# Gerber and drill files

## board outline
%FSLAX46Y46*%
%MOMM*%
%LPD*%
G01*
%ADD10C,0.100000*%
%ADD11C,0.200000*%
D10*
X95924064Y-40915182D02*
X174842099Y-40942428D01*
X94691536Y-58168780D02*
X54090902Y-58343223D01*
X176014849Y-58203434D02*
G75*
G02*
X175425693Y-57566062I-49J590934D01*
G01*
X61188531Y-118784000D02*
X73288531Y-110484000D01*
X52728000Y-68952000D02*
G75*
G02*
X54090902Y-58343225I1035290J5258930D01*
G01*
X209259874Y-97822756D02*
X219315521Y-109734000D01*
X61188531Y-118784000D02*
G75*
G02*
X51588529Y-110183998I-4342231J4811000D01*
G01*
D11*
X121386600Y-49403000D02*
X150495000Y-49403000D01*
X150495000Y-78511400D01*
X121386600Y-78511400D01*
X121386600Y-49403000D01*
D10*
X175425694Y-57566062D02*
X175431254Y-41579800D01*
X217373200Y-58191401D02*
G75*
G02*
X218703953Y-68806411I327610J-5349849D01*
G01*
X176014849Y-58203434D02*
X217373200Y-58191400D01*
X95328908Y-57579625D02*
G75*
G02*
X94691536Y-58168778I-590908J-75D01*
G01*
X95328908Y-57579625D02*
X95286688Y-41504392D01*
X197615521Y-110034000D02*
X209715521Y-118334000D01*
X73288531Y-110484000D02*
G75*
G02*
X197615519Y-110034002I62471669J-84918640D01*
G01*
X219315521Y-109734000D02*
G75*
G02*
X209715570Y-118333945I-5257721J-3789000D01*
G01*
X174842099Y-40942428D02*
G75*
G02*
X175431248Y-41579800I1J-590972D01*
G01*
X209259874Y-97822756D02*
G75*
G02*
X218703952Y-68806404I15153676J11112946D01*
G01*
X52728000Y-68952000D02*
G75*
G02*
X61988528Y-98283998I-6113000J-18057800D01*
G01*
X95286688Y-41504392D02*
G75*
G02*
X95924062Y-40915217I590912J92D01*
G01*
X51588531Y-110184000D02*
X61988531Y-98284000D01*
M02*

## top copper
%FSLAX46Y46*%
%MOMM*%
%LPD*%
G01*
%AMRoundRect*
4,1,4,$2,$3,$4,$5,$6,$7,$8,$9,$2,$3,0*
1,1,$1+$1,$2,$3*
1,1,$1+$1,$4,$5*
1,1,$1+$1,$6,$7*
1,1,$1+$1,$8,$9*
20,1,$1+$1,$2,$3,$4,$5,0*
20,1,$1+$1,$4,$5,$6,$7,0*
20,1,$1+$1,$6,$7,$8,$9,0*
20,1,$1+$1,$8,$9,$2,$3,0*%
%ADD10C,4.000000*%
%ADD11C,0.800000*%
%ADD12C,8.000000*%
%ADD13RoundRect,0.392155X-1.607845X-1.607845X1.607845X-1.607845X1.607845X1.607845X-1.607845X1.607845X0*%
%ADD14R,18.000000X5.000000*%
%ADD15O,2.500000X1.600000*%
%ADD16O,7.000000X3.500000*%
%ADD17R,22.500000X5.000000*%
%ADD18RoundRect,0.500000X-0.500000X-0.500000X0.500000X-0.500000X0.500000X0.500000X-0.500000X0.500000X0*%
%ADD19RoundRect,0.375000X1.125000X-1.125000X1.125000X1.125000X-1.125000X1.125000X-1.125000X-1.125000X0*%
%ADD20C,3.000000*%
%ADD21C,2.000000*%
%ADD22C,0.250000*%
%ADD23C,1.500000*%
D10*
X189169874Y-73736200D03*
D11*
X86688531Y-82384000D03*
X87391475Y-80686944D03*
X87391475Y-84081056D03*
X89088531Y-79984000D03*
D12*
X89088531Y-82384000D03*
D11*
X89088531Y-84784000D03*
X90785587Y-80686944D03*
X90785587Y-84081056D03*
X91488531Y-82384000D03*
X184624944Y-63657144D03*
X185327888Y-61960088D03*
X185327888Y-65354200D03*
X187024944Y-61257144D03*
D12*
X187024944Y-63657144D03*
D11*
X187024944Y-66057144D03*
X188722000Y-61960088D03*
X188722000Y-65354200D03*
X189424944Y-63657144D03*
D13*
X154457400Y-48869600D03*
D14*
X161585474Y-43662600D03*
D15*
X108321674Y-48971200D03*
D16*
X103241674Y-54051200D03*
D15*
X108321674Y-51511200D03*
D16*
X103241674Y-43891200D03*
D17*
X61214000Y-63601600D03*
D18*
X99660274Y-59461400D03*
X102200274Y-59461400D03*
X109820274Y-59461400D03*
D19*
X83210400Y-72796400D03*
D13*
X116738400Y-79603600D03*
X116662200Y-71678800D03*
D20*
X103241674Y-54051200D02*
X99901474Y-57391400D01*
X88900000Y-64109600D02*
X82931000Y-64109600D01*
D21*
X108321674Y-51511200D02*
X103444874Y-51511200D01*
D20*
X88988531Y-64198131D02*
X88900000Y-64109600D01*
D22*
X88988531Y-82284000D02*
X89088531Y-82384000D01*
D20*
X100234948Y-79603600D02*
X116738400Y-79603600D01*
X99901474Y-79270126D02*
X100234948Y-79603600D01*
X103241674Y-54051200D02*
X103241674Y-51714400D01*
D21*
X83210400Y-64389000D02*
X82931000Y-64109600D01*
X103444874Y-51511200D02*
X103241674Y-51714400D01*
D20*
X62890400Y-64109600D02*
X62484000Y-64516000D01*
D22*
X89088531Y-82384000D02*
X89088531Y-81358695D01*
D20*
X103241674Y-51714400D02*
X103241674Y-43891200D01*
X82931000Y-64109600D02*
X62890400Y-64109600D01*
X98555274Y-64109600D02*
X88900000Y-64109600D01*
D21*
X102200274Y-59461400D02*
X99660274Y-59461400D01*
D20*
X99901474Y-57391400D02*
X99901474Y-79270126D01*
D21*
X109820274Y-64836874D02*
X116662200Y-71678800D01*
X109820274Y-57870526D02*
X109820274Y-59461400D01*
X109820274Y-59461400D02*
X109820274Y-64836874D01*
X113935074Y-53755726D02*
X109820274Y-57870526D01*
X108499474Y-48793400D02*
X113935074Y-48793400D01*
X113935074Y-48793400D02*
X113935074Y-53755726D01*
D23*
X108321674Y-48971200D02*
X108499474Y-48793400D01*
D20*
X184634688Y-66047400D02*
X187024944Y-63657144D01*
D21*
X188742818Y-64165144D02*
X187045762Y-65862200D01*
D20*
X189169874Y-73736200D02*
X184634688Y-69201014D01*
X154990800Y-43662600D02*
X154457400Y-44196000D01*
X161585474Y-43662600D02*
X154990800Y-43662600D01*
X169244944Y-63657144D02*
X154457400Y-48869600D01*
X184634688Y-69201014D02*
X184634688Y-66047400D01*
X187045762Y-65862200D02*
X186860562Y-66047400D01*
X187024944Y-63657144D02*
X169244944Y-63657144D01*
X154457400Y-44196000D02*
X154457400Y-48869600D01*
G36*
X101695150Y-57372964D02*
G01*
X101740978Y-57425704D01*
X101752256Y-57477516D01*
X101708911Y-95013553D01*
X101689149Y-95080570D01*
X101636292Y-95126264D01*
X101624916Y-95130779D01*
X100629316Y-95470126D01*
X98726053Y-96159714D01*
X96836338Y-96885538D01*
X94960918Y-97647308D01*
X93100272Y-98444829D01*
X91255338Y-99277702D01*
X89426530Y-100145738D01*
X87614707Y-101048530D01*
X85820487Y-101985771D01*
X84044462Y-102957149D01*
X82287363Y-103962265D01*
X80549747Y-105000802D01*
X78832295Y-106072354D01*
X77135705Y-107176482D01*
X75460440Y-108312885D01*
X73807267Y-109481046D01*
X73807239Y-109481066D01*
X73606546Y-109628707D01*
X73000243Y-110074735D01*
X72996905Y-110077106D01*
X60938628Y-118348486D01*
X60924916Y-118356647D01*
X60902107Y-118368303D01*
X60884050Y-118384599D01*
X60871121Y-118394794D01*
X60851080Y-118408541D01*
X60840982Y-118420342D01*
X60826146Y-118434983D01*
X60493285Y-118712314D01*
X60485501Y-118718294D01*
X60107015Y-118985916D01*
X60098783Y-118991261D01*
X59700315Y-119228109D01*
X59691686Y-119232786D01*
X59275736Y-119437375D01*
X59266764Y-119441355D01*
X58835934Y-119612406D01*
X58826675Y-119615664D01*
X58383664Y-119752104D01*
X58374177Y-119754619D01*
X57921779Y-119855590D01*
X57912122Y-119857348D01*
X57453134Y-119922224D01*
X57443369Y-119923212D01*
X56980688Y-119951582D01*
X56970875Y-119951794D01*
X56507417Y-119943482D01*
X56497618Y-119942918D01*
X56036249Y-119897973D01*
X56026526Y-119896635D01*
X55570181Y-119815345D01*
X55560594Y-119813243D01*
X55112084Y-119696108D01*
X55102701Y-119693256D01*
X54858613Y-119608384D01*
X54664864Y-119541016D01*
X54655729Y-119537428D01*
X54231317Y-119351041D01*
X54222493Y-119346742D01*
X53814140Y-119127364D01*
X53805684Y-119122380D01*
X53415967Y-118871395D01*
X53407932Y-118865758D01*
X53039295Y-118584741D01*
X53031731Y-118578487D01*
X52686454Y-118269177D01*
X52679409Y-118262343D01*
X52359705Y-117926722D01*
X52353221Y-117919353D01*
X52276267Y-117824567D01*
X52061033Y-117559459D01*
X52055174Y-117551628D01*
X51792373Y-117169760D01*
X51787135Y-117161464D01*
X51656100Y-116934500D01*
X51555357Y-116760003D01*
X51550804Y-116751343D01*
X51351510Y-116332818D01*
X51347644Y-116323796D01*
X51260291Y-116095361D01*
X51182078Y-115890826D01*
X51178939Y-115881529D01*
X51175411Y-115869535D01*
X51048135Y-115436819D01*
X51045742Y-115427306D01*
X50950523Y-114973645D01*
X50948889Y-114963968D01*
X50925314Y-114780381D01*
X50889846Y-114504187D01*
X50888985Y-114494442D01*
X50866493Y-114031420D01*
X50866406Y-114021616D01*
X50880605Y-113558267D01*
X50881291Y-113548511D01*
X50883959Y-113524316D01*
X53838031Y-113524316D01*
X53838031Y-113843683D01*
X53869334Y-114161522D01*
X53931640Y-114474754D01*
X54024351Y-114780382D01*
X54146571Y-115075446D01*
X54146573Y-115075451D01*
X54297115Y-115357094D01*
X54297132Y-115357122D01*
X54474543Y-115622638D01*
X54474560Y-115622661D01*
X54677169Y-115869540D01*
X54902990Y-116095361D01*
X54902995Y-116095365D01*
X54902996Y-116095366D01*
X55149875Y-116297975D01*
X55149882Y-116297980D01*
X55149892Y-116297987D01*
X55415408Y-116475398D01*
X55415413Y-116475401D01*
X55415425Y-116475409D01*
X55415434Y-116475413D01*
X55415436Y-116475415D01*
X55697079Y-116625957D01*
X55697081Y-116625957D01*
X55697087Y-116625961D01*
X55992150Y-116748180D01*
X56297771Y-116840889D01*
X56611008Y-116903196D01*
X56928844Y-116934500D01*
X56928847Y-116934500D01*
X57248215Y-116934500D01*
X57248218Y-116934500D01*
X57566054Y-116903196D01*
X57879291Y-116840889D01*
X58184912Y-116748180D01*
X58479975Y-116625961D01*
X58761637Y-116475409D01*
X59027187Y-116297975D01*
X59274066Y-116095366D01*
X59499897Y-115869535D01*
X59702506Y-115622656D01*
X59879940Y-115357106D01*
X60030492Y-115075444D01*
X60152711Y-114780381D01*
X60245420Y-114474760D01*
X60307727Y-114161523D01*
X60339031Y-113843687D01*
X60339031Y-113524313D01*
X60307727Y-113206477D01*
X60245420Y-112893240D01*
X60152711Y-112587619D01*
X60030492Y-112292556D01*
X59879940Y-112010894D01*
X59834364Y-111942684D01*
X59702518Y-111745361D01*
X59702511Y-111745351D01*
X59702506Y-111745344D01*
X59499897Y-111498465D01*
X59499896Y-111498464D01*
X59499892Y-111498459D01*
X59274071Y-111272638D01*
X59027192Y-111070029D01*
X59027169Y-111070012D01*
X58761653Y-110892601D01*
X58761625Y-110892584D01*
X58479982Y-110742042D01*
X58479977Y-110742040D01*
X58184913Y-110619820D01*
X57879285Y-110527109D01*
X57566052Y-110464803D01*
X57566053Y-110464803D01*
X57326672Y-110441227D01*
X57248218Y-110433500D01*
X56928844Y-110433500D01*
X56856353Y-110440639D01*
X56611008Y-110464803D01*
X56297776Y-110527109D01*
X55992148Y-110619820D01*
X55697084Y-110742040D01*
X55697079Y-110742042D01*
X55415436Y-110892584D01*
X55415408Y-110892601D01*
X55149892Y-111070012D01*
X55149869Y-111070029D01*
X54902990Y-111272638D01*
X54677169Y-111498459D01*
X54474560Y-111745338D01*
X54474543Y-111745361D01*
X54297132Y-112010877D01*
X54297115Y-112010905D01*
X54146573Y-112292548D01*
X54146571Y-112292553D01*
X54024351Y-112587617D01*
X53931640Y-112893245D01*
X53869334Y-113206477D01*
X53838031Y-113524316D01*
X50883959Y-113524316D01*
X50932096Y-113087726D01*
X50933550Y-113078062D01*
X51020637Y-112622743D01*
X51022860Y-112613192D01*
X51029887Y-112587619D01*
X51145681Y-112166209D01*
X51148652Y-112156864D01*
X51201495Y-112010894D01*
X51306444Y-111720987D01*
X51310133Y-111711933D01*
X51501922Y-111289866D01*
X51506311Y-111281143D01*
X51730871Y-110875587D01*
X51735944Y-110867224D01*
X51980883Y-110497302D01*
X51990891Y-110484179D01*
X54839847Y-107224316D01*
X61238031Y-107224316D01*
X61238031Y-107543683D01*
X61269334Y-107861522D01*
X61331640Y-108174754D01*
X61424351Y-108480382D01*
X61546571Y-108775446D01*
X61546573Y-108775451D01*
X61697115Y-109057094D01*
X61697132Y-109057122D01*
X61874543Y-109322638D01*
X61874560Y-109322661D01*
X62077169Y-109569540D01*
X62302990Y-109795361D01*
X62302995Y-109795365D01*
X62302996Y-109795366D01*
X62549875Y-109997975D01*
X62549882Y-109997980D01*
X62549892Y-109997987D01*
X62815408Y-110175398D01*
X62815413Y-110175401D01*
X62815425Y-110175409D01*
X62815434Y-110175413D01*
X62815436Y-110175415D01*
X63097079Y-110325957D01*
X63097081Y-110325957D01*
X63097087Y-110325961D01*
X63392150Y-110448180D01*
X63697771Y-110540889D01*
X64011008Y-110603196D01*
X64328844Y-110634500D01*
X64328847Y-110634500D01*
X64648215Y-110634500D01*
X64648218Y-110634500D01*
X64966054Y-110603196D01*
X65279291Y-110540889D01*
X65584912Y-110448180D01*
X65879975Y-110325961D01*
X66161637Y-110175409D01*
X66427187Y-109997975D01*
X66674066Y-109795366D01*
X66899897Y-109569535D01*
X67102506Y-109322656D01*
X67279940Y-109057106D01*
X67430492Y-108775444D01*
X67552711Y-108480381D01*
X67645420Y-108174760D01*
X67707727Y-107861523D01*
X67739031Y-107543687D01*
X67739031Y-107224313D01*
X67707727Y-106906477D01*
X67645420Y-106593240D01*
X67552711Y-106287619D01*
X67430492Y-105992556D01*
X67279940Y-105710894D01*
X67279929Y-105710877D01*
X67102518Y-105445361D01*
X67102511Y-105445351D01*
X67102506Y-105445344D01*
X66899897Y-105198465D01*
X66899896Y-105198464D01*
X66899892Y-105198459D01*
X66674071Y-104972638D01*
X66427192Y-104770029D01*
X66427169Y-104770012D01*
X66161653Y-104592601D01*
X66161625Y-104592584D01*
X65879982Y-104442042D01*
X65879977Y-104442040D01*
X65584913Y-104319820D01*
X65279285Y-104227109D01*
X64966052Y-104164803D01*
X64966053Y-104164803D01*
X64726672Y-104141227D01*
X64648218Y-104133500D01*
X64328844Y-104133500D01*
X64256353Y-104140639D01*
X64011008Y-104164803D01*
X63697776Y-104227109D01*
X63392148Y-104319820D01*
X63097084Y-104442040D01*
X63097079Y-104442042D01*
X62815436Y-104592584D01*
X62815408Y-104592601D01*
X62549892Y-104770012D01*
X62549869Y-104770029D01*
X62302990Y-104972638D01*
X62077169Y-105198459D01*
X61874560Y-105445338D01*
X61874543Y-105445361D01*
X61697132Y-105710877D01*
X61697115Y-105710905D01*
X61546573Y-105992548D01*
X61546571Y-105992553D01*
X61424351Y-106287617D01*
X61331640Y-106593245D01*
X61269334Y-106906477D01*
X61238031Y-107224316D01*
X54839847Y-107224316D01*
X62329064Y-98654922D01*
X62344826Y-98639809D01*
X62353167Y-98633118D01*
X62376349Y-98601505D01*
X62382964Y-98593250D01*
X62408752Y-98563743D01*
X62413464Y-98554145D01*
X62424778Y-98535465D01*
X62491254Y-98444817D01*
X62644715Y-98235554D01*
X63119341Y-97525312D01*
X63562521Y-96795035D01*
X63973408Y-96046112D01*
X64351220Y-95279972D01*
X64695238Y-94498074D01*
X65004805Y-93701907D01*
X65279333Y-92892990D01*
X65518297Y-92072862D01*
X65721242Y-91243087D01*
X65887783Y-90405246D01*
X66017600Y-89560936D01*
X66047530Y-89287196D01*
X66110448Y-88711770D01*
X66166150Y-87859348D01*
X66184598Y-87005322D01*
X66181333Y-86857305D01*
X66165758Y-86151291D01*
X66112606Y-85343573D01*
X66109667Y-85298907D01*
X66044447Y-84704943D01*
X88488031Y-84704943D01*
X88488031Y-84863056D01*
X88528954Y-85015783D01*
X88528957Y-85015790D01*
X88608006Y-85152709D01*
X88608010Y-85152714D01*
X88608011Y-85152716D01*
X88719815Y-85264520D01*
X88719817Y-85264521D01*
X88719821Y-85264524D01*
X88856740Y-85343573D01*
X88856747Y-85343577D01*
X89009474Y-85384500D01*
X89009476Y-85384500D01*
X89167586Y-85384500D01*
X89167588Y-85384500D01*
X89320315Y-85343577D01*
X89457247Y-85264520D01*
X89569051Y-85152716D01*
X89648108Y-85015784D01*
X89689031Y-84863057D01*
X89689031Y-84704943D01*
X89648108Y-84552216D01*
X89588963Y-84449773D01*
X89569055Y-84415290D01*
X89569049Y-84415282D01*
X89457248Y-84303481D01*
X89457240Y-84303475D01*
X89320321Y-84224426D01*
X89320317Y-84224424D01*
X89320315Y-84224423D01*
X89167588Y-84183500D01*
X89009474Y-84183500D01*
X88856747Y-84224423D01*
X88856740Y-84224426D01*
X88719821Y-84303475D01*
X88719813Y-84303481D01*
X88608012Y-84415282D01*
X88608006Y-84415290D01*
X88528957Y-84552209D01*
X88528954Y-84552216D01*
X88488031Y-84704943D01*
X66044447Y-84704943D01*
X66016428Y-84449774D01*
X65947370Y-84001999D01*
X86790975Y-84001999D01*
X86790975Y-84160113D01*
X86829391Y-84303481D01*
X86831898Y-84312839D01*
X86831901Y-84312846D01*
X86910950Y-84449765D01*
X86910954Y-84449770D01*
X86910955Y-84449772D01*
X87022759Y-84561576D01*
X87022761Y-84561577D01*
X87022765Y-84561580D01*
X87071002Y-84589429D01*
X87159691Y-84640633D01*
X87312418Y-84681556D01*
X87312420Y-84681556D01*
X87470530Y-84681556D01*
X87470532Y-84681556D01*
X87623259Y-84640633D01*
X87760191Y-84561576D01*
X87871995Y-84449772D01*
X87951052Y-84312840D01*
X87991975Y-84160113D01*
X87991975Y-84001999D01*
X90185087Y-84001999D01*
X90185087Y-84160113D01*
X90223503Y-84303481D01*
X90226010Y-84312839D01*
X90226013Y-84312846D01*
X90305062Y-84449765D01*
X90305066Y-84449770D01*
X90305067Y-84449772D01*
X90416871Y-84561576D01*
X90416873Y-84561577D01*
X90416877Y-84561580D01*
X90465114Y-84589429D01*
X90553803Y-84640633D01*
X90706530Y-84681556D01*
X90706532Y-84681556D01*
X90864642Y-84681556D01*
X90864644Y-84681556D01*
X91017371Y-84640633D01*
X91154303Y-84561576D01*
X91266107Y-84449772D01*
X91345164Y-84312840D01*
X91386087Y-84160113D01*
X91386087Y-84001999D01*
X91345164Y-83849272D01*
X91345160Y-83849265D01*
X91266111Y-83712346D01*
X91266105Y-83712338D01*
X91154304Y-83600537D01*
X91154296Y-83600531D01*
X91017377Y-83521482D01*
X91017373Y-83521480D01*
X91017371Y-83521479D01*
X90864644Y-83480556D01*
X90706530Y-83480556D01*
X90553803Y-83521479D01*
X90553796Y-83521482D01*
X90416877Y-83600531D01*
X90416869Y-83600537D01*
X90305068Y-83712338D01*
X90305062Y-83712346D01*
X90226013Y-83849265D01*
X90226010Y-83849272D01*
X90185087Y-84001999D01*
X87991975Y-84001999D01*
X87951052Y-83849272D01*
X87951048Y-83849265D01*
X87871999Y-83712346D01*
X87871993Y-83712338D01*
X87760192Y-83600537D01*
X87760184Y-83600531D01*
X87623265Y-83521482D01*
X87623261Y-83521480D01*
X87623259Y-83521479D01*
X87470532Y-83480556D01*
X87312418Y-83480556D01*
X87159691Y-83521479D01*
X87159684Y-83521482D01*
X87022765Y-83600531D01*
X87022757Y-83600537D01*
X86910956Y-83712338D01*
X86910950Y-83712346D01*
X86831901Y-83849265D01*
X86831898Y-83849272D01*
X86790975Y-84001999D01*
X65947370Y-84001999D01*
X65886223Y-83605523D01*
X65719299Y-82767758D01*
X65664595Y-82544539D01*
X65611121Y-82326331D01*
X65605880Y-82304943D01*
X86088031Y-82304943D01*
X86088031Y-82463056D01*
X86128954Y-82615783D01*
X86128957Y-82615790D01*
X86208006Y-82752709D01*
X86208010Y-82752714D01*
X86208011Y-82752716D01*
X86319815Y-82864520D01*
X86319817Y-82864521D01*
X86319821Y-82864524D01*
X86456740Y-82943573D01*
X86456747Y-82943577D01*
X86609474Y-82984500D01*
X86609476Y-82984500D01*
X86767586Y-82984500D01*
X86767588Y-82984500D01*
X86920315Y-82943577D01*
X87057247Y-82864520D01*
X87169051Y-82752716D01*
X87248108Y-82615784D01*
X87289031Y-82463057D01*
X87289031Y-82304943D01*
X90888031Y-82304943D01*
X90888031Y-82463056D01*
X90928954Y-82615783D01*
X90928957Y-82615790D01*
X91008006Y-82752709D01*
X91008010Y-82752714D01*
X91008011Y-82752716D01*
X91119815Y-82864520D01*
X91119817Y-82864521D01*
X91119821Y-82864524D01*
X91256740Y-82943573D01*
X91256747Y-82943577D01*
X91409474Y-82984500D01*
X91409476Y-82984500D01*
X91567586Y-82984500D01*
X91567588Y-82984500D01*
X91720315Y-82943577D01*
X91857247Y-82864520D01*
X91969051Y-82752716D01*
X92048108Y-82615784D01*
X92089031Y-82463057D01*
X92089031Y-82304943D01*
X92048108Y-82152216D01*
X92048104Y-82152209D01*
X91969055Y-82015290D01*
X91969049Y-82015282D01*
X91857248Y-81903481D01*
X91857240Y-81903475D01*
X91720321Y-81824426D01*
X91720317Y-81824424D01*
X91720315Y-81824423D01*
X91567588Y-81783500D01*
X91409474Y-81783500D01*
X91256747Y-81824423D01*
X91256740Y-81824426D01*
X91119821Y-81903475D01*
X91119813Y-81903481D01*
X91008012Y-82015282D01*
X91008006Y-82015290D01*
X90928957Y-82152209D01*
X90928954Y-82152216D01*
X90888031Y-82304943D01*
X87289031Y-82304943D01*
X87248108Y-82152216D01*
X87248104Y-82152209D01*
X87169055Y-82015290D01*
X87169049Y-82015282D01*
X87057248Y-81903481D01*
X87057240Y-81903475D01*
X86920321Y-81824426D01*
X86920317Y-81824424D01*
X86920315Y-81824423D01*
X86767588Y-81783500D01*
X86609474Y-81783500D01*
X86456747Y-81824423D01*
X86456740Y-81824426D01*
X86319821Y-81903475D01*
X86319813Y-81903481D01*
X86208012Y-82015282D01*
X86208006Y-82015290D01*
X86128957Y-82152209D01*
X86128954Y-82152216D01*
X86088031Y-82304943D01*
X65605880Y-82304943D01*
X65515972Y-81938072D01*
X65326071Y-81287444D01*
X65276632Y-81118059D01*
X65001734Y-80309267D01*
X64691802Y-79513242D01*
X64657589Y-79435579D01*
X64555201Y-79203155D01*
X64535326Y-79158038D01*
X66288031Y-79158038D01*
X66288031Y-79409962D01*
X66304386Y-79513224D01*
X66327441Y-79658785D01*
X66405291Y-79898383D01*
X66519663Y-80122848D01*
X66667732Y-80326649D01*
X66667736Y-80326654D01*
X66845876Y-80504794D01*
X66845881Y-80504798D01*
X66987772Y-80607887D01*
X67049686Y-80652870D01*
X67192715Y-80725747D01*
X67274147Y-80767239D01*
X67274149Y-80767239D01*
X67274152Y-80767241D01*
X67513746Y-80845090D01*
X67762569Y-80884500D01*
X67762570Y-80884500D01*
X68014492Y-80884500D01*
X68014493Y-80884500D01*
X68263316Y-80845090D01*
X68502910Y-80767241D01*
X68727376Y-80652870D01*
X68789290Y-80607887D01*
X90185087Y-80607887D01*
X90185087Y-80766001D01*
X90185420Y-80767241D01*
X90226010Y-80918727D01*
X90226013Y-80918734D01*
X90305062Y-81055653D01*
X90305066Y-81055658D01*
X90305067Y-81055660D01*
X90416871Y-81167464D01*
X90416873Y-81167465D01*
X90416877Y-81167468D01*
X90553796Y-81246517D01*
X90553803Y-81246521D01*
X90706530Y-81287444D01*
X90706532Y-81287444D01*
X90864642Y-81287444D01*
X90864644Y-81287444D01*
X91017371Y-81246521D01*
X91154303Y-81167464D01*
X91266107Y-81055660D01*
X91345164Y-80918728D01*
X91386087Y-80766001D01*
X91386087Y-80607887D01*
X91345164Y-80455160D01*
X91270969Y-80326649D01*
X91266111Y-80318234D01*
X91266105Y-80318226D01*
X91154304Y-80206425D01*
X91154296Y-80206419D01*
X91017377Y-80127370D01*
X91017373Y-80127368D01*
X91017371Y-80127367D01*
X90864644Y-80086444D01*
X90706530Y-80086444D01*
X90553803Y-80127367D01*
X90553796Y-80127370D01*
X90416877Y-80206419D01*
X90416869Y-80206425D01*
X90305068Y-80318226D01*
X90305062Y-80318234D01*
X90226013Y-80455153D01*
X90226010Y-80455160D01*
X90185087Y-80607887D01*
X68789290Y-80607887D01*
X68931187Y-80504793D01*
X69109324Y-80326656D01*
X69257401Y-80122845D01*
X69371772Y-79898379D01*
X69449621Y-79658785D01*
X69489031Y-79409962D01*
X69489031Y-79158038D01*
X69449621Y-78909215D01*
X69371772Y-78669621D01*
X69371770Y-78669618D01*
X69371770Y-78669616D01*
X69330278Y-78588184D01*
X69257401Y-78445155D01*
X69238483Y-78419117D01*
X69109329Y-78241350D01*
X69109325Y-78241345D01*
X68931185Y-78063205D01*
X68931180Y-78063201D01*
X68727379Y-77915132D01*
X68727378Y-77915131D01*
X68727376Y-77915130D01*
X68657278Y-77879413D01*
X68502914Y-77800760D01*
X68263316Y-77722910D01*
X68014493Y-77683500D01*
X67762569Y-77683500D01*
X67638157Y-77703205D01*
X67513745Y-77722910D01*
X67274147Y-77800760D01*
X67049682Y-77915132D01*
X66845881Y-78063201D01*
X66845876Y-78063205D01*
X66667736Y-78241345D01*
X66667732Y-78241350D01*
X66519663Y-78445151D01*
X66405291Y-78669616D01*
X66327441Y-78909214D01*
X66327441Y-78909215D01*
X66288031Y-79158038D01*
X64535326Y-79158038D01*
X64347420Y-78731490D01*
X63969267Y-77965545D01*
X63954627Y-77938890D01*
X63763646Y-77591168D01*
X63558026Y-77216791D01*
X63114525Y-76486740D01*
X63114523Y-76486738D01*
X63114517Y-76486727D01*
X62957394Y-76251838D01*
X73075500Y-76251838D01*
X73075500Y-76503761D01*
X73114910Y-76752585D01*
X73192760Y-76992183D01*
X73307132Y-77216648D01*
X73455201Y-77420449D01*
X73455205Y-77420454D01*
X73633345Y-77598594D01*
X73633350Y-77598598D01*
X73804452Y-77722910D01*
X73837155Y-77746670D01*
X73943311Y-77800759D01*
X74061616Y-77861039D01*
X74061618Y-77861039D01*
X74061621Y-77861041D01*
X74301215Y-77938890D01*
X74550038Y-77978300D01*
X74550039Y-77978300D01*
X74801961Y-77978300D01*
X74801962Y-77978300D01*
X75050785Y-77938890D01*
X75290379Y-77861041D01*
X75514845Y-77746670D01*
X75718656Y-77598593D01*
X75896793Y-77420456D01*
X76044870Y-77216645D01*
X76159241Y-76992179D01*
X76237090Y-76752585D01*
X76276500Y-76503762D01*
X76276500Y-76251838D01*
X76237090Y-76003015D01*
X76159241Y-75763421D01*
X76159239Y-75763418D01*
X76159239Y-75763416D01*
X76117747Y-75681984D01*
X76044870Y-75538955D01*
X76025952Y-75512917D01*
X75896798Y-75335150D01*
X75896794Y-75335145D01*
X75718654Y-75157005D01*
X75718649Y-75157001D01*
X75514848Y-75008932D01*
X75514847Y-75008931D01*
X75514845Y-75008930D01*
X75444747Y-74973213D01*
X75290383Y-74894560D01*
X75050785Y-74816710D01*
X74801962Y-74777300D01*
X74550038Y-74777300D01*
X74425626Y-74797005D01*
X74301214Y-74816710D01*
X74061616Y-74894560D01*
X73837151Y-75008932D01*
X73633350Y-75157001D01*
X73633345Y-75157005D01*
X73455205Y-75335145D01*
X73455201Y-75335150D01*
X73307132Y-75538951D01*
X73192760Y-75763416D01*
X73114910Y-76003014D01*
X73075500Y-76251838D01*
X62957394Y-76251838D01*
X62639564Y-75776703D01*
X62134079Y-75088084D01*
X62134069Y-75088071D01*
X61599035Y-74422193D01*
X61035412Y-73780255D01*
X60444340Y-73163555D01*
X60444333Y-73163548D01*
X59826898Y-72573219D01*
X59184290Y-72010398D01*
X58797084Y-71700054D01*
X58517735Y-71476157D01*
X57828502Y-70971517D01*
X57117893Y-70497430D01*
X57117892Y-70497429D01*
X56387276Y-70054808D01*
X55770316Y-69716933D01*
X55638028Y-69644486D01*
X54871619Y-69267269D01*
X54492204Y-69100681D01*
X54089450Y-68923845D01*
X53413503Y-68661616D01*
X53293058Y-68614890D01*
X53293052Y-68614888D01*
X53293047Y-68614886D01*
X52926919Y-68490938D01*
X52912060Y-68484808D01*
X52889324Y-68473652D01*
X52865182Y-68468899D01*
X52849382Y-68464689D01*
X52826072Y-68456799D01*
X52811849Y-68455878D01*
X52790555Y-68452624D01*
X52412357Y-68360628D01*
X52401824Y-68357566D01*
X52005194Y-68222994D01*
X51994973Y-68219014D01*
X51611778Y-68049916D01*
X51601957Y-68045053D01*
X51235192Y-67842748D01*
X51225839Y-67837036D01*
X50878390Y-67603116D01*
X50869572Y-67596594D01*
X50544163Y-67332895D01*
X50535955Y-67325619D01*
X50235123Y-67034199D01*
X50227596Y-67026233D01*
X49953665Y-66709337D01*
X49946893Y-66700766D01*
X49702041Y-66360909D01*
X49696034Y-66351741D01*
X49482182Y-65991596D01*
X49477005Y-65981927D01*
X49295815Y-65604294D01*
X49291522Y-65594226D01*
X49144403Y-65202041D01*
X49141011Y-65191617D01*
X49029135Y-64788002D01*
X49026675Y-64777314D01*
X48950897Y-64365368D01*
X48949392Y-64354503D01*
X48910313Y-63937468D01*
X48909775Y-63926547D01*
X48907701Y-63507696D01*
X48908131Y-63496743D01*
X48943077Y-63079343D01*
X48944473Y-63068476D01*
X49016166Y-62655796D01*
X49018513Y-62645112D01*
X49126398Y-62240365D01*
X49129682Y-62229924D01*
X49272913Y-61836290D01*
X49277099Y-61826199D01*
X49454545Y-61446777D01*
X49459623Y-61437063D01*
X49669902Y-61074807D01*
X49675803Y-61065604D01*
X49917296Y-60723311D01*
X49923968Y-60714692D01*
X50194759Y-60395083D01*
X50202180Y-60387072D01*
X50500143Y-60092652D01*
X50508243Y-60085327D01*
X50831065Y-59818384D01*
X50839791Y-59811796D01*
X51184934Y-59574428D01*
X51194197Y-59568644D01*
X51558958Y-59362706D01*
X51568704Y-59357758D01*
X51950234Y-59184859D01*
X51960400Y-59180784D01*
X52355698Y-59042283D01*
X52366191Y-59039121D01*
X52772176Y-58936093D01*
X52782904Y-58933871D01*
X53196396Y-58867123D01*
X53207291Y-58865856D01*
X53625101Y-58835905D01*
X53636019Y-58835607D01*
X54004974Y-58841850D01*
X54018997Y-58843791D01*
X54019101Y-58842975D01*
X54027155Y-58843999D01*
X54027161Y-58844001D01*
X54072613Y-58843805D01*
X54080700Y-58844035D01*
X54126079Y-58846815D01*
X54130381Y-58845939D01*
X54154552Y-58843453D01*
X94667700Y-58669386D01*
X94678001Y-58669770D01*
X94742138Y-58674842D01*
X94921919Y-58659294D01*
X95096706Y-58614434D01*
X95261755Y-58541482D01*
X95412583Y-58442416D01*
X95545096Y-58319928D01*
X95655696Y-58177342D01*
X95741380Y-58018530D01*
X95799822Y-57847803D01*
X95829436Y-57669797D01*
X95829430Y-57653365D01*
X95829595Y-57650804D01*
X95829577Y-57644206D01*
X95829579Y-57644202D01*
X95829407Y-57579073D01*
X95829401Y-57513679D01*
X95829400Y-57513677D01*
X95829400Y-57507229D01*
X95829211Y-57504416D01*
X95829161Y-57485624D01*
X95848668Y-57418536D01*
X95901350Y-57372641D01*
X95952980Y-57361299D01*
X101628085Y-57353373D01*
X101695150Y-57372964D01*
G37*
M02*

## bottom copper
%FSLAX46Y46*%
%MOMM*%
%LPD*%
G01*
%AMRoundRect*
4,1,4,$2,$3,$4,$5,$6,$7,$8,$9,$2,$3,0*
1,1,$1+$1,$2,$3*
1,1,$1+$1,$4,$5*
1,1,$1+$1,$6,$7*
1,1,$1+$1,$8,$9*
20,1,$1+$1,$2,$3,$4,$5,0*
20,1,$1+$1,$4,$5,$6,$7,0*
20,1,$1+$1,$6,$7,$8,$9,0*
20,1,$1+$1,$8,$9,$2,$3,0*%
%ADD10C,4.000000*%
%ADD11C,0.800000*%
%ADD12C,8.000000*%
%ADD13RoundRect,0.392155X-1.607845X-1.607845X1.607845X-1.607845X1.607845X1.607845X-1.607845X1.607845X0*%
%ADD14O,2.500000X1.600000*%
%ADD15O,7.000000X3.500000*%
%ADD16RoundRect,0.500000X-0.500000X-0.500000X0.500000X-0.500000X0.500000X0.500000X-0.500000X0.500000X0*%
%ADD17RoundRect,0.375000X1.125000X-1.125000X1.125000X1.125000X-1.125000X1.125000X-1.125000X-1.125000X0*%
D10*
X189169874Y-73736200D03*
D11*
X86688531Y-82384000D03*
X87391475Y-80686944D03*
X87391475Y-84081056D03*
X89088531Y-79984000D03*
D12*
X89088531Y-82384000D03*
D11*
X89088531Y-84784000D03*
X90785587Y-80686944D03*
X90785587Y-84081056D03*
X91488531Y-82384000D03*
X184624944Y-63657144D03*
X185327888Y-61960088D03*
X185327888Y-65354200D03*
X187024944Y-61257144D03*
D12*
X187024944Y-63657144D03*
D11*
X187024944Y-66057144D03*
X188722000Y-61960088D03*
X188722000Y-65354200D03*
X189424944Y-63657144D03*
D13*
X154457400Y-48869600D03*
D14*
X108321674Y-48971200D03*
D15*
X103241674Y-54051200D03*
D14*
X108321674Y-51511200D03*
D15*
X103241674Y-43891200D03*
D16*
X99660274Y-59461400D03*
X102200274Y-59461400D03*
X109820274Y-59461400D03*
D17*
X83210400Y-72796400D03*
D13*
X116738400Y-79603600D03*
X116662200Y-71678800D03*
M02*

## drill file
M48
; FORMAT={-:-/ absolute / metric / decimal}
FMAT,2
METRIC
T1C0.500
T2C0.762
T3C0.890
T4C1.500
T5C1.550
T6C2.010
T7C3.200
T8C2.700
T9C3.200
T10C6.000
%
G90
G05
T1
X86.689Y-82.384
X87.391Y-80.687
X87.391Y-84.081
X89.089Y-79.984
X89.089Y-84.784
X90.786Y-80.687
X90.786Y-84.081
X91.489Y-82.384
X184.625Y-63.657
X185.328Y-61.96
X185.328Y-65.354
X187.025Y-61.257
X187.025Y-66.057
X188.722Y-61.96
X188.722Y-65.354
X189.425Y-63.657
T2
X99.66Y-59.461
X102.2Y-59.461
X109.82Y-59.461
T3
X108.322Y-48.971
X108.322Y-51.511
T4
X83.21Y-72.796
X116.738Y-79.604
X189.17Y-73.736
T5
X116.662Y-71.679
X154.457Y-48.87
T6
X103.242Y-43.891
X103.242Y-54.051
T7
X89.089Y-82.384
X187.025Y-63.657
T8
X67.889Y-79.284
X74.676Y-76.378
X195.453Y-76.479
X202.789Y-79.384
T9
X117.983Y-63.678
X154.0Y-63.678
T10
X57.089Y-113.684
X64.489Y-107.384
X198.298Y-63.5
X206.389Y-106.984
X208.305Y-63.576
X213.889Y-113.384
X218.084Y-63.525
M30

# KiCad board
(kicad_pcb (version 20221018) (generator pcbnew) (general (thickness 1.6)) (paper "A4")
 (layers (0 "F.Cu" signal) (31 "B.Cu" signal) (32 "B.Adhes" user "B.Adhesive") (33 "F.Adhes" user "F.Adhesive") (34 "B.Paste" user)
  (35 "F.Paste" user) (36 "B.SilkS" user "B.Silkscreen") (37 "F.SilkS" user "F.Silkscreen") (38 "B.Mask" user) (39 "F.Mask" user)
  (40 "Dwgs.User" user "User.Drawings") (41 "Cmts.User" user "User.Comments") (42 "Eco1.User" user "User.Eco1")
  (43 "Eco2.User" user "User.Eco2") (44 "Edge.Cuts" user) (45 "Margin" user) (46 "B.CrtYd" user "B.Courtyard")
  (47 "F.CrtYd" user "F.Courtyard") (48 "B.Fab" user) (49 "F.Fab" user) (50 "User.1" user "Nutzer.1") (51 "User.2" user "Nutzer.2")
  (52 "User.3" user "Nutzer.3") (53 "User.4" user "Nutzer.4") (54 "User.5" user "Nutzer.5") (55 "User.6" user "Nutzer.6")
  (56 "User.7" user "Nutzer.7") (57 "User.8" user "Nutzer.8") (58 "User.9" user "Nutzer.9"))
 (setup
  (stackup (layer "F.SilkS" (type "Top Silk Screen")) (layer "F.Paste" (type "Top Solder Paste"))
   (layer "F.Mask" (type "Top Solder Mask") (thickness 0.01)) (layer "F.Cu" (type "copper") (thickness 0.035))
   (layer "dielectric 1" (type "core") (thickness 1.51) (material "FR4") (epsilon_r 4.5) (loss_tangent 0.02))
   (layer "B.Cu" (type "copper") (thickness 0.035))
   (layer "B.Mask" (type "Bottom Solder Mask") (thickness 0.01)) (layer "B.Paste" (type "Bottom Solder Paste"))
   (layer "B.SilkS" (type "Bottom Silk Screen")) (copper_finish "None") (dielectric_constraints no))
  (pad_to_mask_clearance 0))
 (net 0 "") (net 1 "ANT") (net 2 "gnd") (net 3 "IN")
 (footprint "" (layer "F.Cu") (at 189.169874 73.7362)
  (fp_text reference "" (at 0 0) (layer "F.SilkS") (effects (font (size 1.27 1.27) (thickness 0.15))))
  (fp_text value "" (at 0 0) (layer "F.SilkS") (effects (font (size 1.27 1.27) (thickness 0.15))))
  (pad "1" thru_hole circle (at 0 0 90) (size 4 4) (drill 1.5) (layers "*.Cu" "*.Mask") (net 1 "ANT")))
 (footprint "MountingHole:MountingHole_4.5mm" (layer "F.Cu") (at 218.0844 63.5254)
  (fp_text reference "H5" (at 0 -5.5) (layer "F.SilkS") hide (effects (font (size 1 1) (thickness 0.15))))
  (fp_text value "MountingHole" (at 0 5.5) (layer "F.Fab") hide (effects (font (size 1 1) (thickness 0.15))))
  (pad "" np_thru_hole circle (at 0 0) (size 6 6) (drill 6) (layers "F&B.Cu" "*.Mask")))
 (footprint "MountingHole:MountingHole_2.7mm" (layer "F.Cu") (at 195.453 76.4794)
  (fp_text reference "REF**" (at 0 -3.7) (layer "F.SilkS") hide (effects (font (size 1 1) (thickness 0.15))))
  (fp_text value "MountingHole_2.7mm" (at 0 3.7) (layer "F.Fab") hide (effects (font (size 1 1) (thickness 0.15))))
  (pad "" np_thru_hole circle (at 0 0) (size 2.7 2.7) (drill 2.7) (layers "F&B.Cu" "*.Mask")))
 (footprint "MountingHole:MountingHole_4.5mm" (layer "F.Cu") (at 198.2978 63.5)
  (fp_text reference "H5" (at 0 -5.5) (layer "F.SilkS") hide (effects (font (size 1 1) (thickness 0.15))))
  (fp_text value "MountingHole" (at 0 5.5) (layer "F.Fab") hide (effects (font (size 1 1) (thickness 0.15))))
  (pad "" np_thru_hole circle (at 0 0) (size 6 6) (drill 6) (layers "F&B.Cu" "*.Mask")))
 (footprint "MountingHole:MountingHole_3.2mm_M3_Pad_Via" (layer "F.Cu") (at 89.088531 82.384)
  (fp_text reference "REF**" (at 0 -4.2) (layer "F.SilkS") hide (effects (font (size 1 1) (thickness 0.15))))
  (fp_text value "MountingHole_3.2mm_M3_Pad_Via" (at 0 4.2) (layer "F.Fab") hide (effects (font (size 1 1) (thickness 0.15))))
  (pad "1" thru_hole circle (at -2.4 0) (size 0.8 0.8) (drill 0.5) (layers "*.Cu" "*.Mask"))
  (pad "1" thru_hole circle (at -1.697056 -1.697056) (size 0.8 0.8) (drill 0.5) (layers "*.Cu" "*.Mask") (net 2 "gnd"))
  (pad "1" thru_hole circle (at -1.697056 1.697056) (size 0.8 0.8) (drill 0.5) (layers "*.Cu" "*.Mask"))
  (pad "1" thru_hole circle (at 0 -2.4) (size 0.8 0.8) (drill 0.5) (layers "*.Cu" "*.Mask") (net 2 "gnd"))
  (pad "1" thru_hole circle (at 0 0) (size 8 8) (drill 3.2) (layers "*.Cu" "*.Mask") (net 2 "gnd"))
  (pad "1" thru_hole circle (at 0 2.4) (size 0.8 0.8) (drill 0.5) (layers "*.Cu" "*.Mask"))
  (pad "1" thru_hole circle (at 1.697056 -1.697056) (size 0.8 0.8) (drill 0.5) (layers "*.Cu" "*.Mask"))
  (pad "1" thru_hole circle (at 1.697056 1.697056) (size 0.8 0.8) (drill 0.5) (layers "*.Cu" "*.Mask"))
  (pad "1" thru_hole circle (at 2.4 0) (size 0.8 0.8) (drill 0.5) (layers "*.Cu" "*.Mask")))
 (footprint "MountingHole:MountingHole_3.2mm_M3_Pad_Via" (layer "F.Cu") (at 187.024944 63.657144)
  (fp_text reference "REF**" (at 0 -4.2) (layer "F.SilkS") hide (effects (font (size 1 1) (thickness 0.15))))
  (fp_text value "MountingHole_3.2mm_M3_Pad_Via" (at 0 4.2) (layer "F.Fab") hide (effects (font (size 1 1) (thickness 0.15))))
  (pad "1" thru_hole circle (at -2.4 0) (size 0.8 0.8) (drill 0.5) (layers "*.Cu" "*.Mask") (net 1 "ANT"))
  (pad "1" thru_hole circle (at -1.697056 -1.697056) (size 0.8 0.8) (drill 0.5) (layers "*.Cu" "*.Mask") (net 1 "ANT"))
  (pad "1" thru_hole circle (at -1.697056 1.697056) (size 0.8 0.8) (drill 0.5) (layers "*.Cu" "*.Mask") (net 1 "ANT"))
  (pad "1" thru_hole circle (at 0 -2.4) (size 0.8 0.8) (drill 0.5) (layers "*.Cu" "*.Mask") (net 1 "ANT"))
  (pad "1" thru_hole circle (at 0 0) (size 8 8) (drill 3.2) (layers "*.Cu" "*.Mask") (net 1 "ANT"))
  (pad "1" thru_hole circle (at 0 2.4) (size 0.8 0.8) (drill 0.5) (layers "*.Cu" "*.Mask") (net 1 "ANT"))
  (pad "1" thru_hole circle (at 1.697056 -1.697056) (size 0.8 0.8) (drill 0.5) (layers "*.Cu" "*.Mask") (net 1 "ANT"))
  (pad "1" thru_hole circle (at 1.697056 1.697056) (size 0.8 0.8) (drill 0.5) (layers "*.Cu" "*.Mask") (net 1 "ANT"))
  (pad "1" thru_hole circle (at 2.4 0) (size 0.8 0.8) (drill 0.5) (layers "*.Cu" "*.Mask") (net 1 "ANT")))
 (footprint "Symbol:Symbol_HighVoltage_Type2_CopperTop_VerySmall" (layer "F.Cu") (at 193.0146 68.072)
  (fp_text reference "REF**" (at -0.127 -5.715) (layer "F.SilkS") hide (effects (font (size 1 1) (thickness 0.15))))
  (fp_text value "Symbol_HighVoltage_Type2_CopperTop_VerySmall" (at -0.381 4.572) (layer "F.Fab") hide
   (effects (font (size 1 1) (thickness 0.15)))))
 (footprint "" (layer "F.Cu") (at 154.4574 48.8696)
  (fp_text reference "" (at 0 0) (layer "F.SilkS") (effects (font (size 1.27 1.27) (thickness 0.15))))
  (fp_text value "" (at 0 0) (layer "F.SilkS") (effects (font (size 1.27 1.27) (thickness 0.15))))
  (pad "5" thru_hole roundrect (at 0 0) (size 4 4) (drill 1.55) (layers "*.Cu" "*.Mask") (roundrect_rratio 0.09803875) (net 1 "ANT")))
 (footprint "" (layer "F.Cu") (at 154.0002 63.6778)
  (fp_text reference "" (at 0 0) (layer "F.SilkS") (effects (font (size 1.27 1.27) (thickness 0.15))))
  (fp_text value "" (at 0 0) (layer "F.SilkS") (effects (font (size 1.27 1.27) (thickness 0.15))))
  (pad "" np_thru_hole circle (at 0 0) (size 3.2 3.2) (drill 3.2) (layers "*.Cu" "*.Mask")))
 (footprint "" (layer "F.Cu") (at 161.585474 43.6626)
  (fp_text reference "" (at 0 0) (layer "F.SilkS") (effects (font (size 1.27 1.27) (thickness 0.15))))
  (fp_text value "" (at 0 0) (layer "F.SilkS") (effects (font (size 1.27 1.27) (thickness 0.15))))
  (pad "1" smd rect (at 0 0) (size 18 5) (layers "F.Cu" "F.Mask") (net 1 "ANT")))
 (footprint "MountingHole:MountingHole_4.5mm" (layer "F.Cu") (at 208.3054 63.5762)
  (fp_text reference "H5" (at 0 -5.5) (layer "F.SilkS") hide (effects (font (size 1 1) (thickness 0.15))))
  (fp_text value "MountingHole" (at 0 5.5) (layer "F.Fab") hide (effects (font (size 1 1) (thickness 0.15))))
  (pad "" np_thru_hole circle (at 0 0) (size 6 6) (drill 6) (layers "F&B.Cu" "*.Mask")))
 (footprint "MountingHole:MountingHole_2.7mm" (layer "F.Cu") (at 74.676 76.3778)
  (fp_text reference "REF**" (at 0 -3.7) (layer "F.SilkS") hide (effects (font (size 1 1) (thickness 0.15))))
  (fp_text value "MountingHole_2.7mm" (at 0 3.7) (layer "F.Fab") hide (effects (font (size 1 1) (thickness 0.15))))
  (pad "" np_thru_hole circle (at 0 0) (size 2.7 2.7) (drill 2.7) (layers "F&B.Cu" "*.Mask")))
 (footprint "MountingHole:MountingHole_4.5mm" (layer "F.Cu") (at 57.088531 113.684)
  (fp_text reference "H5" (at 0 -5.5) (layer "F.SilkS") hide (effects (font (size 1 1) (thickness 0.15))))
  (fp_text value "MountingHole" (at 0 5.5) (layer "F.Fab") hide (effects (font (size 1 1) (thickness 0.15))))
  (pad "" np_thru_hole circle (at 0 0) (size 6 6) (drill 6) (layers "F&B.Cu" "*.Mask")))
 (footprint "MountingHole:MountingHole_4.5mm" (layer "F.Cu") (at 64.488531 107.384)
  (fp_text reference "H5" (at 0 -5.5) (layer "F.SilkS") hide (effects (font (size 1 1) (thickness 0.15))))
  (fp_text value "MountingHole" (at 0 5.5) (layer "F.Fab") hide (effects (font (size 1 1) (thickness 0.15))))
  (pad "" np_thru_hole circle (at 0 0) (size 6 6) (drill 6) (layers "F&B.Cu" "*.Mask")))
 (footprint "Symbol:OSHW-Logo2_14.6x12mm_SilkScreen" (layer "F.Cu") (at 76.588531 90.284)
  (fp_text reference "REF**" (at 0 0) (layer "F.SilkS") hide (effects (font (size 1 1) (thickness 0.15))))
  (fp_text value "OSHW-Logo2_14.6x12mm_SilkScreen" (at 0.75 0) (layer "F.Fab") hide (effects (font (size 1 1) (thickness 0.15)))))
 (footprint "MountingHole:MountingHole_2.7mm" (layer "F.Cu") (at 67.888531 79.284)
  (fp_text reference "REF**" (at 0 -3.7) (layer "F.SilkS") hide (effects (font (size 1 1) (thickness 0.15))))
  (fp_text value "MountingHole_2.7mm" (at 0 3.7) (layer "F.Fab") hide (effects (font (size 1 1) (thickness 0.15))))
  (pad "" np_thru_hole circle (at 0 0) (size 2.7 2.7) (drill 2.7) (layers "F&B.Cu" "*.Mask")))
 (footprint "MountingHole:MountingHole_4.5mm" (layer "F.Cu") (at 206.388531 106.984)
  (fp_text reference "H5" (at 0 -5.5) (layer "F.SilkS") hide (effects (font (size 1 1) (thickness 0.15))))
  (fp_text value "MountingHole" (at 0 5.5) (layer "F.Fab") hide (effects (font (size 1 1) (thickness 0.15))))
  (pad "" np_thru_hole circle (at 0 0) (size 6 6) (drill 6) (layers "F&B.Cu" "*.Mask")))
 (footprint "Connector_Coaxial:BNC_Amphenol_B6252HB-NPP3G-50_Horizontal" (layer "F.Cu") (at 108.321674 48.9712 90)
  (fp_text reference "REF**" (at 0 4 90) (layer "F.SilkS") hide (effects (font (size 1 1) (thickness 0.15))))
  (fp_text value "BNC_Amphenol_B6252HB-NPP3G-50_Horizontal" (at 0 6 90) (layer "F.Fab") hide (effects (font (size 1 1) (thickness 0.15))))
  (pad "1" thru_hole oval (at 0 0 90) (size 1.6 2.5) (drill 0.89) (layers "*.Cu" "*.Mask") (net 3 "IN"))
  (pad "2" thru_hole oval (at -5.08 -5.08 90) (size 3.5 7) (drill 2.01) (layers "*.Cu" "*.Mask") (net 2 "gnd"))
  (pad "2" thru_hole oval (at -2.54 0 90) (size 1.6 2.5) (drill 0.89) (layers "*.Cu" "*.Mask") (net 2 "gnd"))
  (pad "2" thru_hole oval (at 5.08 -5.08 90) (size 3.5 7) (drill 2.01) (layers "*.Cu" "*.Mask") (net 2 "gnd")))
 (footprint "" (layer "F.Cu") (at 61.214 63.6016)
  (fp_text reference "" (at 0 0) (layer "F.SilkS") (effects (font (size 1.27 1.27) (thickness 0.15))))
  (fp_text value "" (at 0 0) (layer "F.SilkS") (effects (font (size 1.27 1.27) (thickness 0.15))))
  (pad "1" smd rect (at 0 0 180) (size 22.5 5) (layers "F.Cu" "F.Mask") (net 2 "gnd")))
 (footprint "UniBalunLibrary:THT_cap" (layer "F.Cu") (at 104.740274 59.4614)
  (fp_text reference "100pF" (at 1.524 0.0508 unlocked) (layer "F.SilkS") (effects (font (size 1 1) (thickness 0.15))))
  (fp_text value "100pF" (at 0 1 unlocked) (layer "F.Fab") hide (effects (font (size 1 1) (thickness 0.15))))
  (pad "1" thru_hole roundrect (at -5.08 0) (size 2 2) (drill 0.762) (layers "*.Cu" "*.Mask") (roundrect_rratio 0.25) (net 2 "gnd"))
  (pad "1" thru_hole roundrect (at -2.54 0) (size 2 2) (drill 0.762) (layers "*.Cu" "*.Mask") (roundrect_rratio 0.25) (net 2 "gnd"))
  (pad "2" thru_hole roundrect (at 5.08 0) (size 2 2) (drill 0.762) (layers "*.Cu" "*.Mask") (roundrect_rratio 0.25) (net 3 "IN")))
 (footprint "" (layer "F.Cu") (at 83.2104 72.7964)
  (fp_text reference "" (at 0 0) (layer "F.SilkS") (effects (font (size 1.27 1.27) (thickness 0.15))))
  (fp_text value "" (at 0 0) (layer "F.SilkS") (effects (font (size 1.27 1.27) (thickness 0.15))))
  (pad "1" thru_hole roundrect (at 0 0 90) (size 3 3) (drill 1.5) (layers "*.Cu" "*.Mask") (roundrect_rratio 0.125) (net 2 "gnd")))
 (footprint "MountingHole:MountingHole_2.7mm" (layer "F.Cu") (at 202.788531 79.384)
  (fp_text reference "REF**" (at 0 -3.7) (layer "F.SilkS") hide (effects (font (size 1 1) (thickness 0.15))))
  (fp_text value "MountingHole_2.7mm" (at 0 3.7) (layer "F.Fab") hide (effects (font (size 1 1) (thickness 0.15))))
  (pad "" np_thru_hole circle (at 0 0) (size 2.7 2.7) (drill 2.7) (layers "F&B.Cu" "*.Mask")))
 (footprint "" (layer "F.Cu") (at 117.983 63.6778)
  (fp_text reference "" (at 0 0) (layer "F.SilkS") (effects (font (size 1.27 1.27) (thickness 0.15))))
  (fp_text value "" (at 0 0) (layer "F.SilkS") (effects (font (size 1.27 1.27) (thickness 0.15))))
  (pad "" np_thru_hole circle (at 0 0) (size 3.2 3.2) (drill 3.2) (layers "F&B.Cu" "*.Mask")))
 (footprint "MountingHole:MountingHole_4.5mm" (layer "F.Cu") (at 213.888531 113.384)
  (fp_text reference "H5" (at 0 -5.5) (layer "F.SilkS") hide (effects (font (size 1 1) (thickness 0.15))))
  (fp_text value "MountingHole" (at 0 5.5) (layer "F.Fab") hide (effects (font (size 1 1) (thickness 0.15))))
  (pad "" np_thru_hole circle (at 0 0) (size 6 6) (drill 6) (layers "F&B.Cu" "*.Mask")))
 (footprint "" (layer "F.Cu") (at 116.7384 79.6036)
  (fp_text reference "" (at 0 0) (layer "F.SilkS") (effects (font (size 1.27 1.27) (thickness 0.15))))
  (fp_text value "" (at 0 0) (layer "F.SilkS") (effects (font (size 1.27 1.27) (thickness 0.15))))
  (pad "5" thru_hole roundrect (at 0 0) (size 4 4) (drill 1.5) (layers "*.Cu" "*.Mask") (roundrect_rratio 0.09803875) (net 2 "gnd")))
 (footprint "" (layer "F.Cu") (at 116.6622 71.6788)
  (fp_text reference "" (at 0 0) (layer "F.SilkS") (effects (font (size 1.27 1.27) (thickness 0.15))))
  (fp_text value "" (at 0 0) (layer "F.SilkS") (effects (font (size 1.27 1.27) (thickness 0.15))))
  (pad "1" thru_hole roundrect (at 0 0) (size 4 4) (drill 1.55) (layers "*.Cu" "*.Mask") (roundrect_rratio 0.09803875) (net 3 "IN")))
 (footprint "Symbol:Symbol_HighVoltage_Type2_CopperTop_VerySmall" (layer "B.Cu") (at 193.0654 68.1482 180)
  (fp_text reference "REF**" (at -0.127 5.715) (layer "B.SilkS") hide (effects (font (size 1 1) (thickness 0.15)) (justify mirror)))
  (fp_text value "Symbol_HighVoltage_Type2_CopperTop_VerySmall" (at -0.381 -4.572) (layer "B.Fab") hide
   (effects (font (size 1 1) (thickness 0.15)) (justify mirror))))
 (gr_line (start 95.924064 40.915182) (end 174.842099 40.942428) (stroke (width 0.1) (type solid)) (layer "Edge.Cuts"))
 (gr_line (start 94.691536 58.16878) (end 54.090902 58.343223) (stroke (width 0.1) (type default)) (layer "Edge.Cuts"))
 (gr_arc (start 176.014849 58.203434) (mid 175.580837 58.013619) (end 175.425694 57.566062) (stroke (width 0.1) (type solid))
  (layer "Edge.Cuts"))
 (gr_line (start 61.188531 118.784) (end 73.288531 110.484) (stroke (width 0.1) (type solid)) (layer "Edge.Cuts"))
 (gr_arc (start 52.728 68.952) (mid 48.447115 63.010103) (end 54.090902 58.343223) (stroke (width 0.1) (type default)) (layer "Edge.Cuts"))
 (gr_line (start 209.259874 97.822756) (end 219.315521 109.734) (stroke (width 0.1) (type solid)) (layer "Edge.Cuts"))
 (gr_arc (start 61.188531 118.784) (mid 52.522011 118.800115) (end 51.588531 110.184) (stroke (width 0.1) (type solid)) (layer "Edge.Cuts"))
 (gr_rect (start 121.3866 49.403) (end 150.495 78.5114) (stroke (width 0.2) (type default)) (fill none) (layer "Edge.Cuts"))
 (gr_line (start 175.425694 57.566062) (end 175.431254 41.5798) (stroke (width 0.1) (type solid)) (layer "Edge.Cuts"))
 (gr_arc (start 217.3732 58.191401) (mid 223.019048 62.874524) (end 218.703952 68.806403) (stroke (width 0.1) (type default))
  (layer "Edge.Cuts"))
 (gr_line (start 176.014849 58.203434) (end 217.3732 58.1914) (stroke (width 0.1) (type default)) (layer "Edge.Cuts"))
 (gr_arc (start 95.328908 57.579625) (mid 95.139087 58.013631) (end 94.691536 58.16878) (stroke (width 0.1) (type solid))
  (layer "Edge.Cuts"))
 (gr_line (start 95.328908 57.579625) (end 95.286688 41.504392) (stroke (width 0.1) (type solid)) (layer "Edge.Cuts"))
 (gr_line (start 197.615521 110.034) (end 209.715521 118.334) (stroke (width 0.1) (type solid)) (layer "Edge.Cuts"))
 (gr_arc (start 73.288531 110.484) (mid 135.37863 89.980918) (end 197.615521 110.034) (stroke (width 0.1) (type solid)) (layer "Edge.Cuts"))
 (gr_arc (start 219.315521 109.734) (mid 218.382028 118.350151) (end 209.715521 118.334) (stroke (width 0.1) (type solid))
  (layer "Edge.Cuts"))
 (gr_arc (start 174.842099 40.942428) (mid 175.276096 41.132256) (end 175.431254 41.5798) (stroke (width 0.1) (type solid))
  (layer "Edge.Cuts"))
 (gr_arc (start 209.259874 97.822756) (mid 206.544408 80.893863) (end 218.703952 68.806403) (stroke (width 0.1) (type solid))
  (layer "Edge.Cuts"))
 (gr_arc (start 52.728 68.952) (mid 64.794913 81.270144) (end 61.988531 98.284) (stroke (width 0.1) (type solid)) (layer "Edge.Cuts"))
 (gr_arc (start 95.286688 41.504392) (mid 95.476504 41.070372) (end 95.92406 40.915237) (stroke (width 0.1) (type solid))
  (layer "Edge.Cuts"))
 (gr_line (start 51.588531 110.184) (end 61.988531 98.284) (stroke (width 0.1) (type solid)) (layer "Edge.Cuts"))
 (segment (start 103.241674 54.0512) (end 99.901474 57.3914) (width 3) (layer "F.Cu") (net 2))
 (segment (start 88.9 64.1096) (end 82.931 64.1096) (width 3) (layer "F.Cu") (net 2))
 (segment (start 108.321674 51.5112) (end 103.444874 51.5112) (width 2) (layer "F.Cu") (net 2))
 (segment (start 88.988531 64.198131) (end 88.9 64.1096) (width 3) (layer "F.Cu") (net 2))
 (segment (start 88.988531 82.284) (end 89.088531 82.384) (width 0.25) (layer "F.Cu") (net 2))
 (segment (start 100.234948 79.6036) (end 116.7384 79.6036) (width 3) (layer "F.Cu") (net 2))
 (segment (start 99.901474 79.270126) (end 100.234948 79.6036) (width 3) (layer "F.Cu") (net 2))
 (segment (start 103.241674 54.0512) (end 103.241674 51.7144) (width 3) (layer "F.Cu") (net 2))
 (segment (start 83.2104 64.389) (end 82.931 64.1096) (width 2) (layer "F.Cu") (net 2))
 (segment (start 103.444874 51.5112) (end 103.241674 51.7144) (width 2) (layer "F.Cu") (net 2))
 (segment (start 62.8904 64.1096) (end 62.484 64.516) (width 3) (layer "F.Cu") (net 2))
 (segment (start 89.088531 82.384) (end 89.088531 81.358695) (width 0.25) (layer "F.Cu") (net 2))
 (segment (start 103.241674 51.7144) (end 103.241674 43.8912) (width 3) (layer "F.Cu") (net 2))
 (segment (start 82.931 64.1096) (end 62.8904 64.1096) (width 3) (layer "F.Cu") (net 2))
 (segment (start 98.555274 64.1096) (end 88.9 64.1096) (width 3) (layer "F.Cu") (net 2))
 (segment (start 102.200274 59.4614) (end 99.660274 59.4614) (width 2) (layer "F.Cu") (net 2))
 (segment (start 99.901474 57.3914) (end 99.901474 79.270126) (width 3) (layer "F.Cu") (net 2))
 (segment (start 109.820274 64.836874) (end 116.6622 71.6788) (width 2) (layer "F.Cu") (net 3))
 (segment (start 109.820274 57.870526) (end 109.820274 59.4614) (width 2) (layer "F.Cu") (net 3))
 (segment (start 109.820274 59.4614) (end 109.820274 64.836874) (width 2) (layer "F.Cu") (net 3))
 (segment (start 113.935074 53.755726) (end 109.820274 57.870526) (width 2) (layer "F.Cu") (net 3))
 (segment (start 108.499474 48.7934) (end 113.935074 48.7934) (width 2) (layer "F.Cu") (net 3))
 (segment (start 113.935074 48.7934) (end 113.935074 53.755726) (width 2) (layer "F.Cu") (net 3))
 (segment (start 108.321674 48.9712) (end 108.499474 48.7934) (width 1.5) (layer "F.Cu") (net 3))
 (segment (start 184.634688 66.0474) (end 187.024944 63.657144) (width 3) (layer "F.Cu") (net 1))
 (segment (start 188.742818 64.165144) (end 187.045762 65.8622) (width 2) (layer "F.Cu") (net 1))
 (segment (start 189.169874 73.7362) (end 184.634688 69.201014) (width 3) (layer "F.Cu") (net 1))
 (segment (start 154.9908 43.6626) (end 154.4574 44.196) (width 3) (layer "F.Cu") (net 1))
 (segment (start 161.585474 43.6626) (end 154.9908 43.6626) (width 3) (layer "F.Cu") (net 1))
 (segment (start 169.244944 63.657144) (end 154.4574 48.8696) (width 3) (layer "F.Cu") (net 1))
 (segment (start 184.634688 69.201014) (end 184.634688 66.0474) (width 3) (layer "F.Cu") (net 1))
 (segment (start 187.045762 65.8622) (end 186.860562 66.0474) (width 3) (layer "F.Cu") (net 1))
 (segment (start 187.024944 63.657144) (end 169.244944 63.657144) (width 3) (layer "F.Cu") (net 1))
 (segment (start 154.4574 44.196) (end 154.4574 48.8696) (width 3) (layer "F.Cu") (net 1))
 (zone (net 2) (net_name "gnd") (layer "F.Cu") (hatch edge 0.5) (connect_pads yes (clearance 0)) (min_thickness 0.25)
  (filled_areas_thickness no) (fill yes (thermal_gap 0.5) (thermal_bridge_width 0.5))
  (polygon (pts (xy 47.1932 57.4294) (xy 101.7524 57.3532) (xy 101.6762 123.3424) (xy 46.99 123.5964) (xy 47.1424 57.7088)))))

